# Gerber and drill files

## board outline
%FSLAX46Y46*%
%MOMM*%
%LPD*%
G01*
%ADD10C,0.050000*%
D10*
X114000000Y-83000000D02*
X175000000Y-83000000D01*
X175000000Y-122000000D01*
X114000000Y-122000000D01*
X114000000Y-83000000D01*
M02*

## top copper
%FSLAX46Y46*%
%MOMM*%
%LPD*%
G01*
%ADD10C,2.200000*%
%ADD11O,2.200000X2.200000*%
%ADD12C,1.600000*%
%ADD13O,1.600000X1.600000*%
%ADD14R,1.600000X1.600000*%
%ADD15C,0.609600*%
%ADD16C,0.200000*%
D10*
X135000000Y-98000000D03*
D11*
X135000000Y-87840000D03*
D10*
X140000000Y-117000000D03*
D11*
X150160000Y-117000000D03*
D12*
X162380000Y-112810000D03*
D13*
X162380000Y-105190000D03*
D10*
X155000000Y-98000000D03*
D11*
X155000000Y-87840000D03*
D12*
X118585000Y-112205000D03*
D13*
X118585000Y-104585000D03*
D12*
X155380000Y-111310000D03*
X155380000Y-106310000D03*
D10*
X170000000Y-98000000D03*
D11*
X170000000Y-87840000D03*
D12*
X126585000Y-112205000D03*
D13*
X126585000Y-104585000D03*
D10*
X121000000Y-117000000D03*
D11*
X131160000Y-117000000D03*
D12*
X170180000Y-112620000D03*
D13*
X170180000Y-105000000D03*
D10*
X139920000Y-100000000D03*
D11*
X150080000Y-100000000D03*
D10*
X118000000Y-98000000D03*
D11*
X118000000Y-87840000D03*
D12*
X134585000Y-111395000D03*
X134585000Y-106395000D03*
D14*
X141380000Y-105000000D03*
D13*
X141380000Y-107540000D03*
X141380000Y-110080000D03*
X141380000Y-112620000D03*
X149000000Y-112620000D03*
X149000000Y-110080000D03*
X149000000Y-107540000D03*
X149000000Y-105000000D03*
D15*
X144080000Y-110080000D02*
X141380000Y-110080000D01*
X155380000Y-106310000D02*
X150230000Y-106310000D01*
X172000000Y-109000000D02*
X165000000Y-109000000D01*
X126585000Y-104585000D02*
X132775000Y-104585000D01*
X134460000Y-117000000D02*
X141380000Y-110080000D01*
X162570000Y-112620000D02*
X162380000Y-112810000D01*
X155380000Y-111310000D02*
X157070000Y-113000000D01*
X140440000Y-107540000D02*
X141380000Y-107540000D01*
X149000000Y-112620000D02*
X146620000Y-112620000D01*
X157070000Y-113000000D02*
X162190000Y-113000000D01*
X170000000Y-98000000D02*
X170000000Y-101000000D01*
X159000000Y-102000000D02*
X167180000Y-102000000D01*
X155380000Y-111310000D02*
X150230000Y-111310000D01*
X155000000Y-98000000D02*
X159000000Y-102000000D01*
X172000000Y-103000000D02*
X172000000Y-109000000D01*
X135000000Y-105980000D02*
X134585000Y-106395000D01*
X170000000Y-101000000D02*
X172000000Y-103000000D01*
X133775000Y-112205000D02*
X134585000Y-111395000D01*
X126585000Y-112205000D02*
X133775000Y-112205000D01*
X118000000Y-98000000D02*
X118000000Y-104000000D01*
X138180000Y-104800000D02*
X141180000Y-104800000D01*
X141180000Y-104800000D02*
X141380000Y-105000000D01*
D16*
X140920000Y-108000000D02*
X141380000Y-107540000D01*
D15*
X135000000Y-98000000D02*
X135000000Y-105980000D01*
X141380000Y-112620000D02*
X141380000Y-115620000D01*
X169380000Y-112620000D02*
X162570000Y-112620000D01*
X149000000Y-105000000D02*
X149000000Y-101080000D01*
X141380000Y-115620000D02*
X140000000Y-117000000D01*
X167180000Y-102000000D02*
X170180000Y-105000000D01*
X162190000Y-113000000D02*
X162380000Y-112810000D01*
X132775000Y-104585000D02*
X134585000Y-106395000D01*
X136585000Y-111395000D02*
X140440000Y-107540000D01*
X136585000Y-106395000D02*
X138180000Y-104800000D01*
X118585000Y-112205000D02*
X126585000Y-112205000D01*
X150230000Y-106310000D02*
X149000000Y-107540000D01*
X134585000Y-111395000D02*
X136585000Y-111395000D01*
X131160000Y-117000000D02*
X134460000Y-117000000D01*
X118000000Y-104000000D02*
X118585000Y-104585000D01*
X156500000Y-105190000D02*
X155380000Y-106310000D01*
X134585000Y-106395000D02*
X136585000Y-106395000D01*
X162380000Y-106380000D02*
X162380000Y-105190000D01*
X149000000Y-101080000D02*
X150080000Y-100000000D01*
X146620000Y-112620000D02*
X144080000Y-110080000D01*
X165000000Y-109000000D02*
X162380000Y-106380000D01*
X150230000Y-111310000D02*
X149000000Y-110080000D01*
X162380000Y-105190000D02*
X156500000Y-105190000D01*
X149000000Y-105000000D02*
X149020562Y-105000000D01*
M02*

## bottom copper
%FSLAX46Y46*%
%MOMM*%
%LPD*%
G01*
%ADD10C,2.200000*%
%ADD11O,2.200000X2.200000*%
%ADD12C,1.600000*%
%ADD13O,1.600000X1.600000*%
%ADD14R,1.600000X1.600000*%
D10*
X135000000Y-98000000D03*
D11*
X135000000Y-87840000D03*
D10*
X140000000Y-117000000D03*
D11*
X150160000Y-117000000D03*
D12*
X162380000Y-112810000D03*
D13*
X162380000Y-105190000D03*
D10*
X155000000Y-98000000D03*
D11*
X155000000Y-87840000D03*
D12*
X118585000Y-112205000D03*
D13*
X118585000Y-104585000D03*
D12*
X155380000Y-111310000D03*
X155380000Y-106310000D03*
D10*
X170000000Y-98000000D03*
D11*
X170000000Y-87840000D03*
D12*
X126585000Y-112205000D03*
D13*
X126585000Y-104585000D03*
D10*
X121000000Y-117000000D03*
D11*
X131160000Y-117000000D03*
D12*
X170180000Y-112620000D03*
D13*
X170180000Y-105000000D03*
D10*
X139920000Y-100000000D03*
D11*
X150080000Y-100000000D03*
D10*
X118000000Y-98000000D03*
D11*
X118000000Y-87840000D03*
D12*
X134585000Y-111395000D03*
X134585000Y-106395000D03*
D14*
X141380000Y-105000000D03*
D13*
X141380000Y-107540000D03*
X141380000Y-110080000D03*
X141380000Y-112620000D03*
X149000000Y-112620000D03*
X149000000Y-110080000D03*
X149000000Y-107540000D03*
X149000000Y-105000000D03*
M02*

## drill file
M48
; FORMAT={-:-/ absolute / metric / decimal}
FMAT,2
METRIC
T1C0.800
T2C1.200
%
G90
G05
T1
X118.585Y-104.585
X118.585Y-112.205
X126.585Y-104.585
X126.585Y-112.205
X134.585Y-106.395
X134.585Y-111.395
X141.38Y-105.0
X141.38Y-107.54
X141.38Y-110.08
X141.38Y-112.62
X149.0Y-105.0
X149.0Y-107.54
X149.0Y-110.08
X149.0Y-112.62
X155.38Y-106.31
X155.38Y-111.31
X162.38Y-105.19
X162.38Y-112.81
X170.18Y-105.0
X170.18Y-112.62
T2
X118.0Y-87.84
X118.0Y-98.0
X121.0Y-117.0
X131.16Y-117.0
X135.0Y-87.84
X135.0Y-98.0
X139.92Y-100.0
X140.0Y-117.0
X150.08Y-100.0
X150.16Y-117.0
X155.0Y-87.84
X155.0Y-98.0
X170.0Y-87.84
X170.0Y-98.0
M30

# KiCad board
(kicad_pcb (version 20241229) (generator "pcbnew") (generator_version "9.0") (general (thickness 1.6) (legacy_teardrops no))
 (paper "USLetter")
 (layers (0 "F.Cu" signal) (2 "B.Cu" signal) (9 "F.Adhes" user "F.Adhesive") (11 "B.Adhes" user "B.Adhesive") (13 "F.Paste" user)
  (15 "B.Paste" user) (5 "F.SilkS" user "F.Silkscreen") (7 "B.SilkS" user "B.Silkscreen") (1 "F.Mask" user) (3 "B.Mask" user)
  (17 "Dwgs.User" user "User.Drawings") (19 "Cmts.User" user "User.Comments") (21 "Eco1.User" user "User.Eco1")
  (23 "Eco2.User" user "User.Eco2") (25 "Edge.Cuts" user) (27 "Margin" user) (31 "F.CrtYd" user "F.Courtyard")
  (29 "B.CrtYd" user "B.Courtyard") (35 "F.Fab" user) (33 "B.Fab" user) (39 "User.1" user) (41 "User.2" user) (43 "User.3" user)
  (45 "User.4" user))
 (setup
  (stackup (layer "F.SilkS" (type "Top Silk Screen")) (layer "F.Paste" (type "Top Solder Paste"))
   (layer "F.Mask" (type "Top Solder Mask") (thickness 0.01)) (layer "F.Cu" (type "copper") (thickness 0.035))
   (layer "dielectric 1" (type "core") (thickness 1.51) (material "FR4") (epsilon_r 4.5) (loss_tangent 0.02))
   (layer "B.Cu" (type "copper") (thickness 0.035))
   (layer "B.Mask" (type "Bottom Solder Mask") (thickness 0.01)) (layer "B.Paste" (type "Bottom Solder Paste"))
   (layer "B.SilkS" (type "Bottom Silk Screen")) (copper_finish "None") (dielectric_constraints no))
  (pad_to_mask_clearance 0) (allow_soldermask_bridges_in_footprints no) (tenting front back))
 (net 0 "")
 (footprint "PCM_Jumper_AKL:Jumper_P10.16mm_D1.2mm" (layer "F.Cu") (at 135 98 90)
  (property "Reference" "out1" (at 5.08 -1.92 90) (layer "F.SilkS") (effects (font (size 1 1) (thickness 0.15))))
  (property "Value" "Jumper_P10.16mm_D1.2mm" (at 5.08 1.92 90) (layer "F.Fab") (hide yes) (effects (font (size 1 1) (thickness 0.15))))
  (pad "1" thru_hole circle (at 0 0 90) (size 2.2 2.2) (drill 1.2) (layers "*.Cu" "*.Mask") (remove_unused_layers no))
  (pad "2" thru_hole oval (at 10.16 0 90) (size 2.2 2.2) (drill 1.2) (layers "*.Cu" "*.Mask") (remove_unused_layers no)))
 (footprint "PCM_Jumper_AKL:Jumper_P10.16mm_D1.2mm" (layer "F.Cu") (at 140 117)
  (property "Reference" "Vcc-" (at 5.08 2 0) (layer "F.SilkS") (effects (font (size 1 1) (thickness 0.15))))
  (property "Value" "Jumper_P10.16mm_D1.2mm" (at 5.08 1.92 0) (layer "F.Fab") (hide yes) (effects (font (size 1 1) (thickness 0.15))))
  (pad "1" thru_hole circle (at 0 0) (size 2.2 2.2) (drill 1.2) (layers "*.Cu" "*.Mask") (remove_unused_layers no))
  (pad "2" thru_hole oval (at 10.16 0) (size 2.2 2.2) (drill 1.2) (layers "*.Cu" "*.Mask") (remove_unused_layers no)))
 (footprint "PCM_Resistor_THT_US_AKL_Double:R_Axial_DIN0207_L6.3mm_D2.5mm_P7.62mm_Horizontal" (layer "F.Cu") (at 162.38 112.81 90)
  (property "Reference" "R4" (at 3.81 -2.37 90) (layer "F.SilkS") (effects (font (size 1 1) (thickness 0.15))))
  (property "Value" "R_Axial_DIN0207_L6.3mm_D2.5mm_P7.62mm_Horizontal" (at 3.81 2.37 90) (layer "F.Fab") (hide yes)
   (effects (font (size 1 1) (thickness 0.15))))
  (pad "1" thru_hole circle (at 0 0 90) (size 1.6 1.6) (drill 0.8) (layers "*.Cu" "*.Mask") (remove_unused_layers no))
  (pad "2" thru_hole oval (at 7.62 0 90) (size 1.6 1.6) (drill 0.8) (layers "*.Cu" "*.Mask") (remove_unused_layers no)))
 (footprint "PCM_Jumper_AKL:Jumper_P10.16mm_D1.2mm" (layer "F.Cu") (at 155 98 90)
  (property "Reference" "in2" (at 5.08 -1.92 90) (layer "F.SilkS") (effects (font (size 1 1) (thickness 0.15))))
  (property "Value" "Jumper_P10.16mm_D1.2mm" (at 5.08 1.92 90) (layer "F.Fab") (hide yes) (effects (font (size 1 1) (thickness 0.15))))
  (pad "1" thru_hole circle (at 0 0 90) (size 2.2 2.2) (drill 1.2) (layers "*.Cu" "*.Mask") (remove_unused_layers no))
  (pad "2" thru_hole oval (at 10.16 0 90) (size 2.2 2.2) (drill 1.2) (layers "*.Cu" "*.Mask") (remove_unused_layers no)))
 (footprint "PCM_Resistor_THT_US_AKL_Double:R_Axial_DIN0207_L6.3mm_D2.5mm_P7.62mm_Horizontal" (layer "F.Cu") (at 118.585 112.205 90)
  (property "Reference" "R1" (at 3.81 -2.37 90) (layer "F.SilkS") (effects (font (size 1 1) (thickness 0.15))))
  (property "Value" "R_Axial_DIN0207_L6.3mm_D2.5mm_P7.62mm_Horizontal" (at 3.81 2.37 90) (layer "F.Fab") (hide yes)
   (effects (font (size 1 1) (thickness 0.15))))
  (pad "1" thru_hole circle (at 0 0 90) (size 1.6 1.6) (drill 0.8) (layers "*.Cu" "*.Mask") (remove_unused_layers no))
  (pad "2" thru_hole oval (at 7.62 0 90) (size 1.6 1.6) (drill 0.8) (layers "*.Cu" "*.Mask") (remove_unused_layers no)))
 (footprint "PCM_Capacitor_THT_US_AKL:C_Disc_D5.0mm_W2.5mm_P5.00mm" (layer "F.Cu") (at 155.38 111.31 90)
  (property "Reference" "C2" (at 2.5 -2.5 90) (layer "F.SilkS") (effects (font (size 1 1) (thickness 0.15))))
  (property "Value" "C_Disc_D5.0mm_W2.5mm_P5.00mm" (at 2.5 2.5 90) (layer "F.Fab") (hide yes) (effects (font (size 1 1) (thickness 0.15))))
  (pad "1" thru_hole circle (at 0 0 90) (size 1.6 1.6) (drill 0.8) (layers "*.Cu" "*.Mask") (remove_unused_layers no))
  (pad "2" thru_hole circle (at 5 0 90) (size 1.6 1.6) (drill 0.8) (layers "*.Cu" "*.Mask") (remove_unused_layers no)))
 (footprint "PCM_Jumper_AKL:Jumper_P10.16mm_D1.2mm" (layer "F.Cu") (at 170 98 90)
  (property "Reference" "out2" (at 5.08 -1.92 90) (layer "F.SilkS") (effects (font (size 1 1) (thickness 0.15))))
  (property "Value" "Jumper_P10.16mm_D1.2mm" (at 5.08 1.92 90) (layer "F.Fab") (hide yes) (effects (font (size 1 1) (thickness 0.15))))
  (pad "1" thru_hole circle (at 0 0 90) (size 2.2 2.2) (drill 1.2) (layers "*.Cu" "*.Mask") (remove_unused_layers no))
  (pad "2" thru_hole oval (at 10.16 0 90) (size 2.2 2.2) (drill 1.2) (layers "*.Cu" "*.Mask") (remove_unused_layers no)))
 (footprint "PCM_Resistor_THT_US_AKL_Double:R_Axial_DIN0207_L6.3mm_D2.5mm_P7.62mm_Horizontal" (layer "F.Cu") (at 126.585 112.205 90)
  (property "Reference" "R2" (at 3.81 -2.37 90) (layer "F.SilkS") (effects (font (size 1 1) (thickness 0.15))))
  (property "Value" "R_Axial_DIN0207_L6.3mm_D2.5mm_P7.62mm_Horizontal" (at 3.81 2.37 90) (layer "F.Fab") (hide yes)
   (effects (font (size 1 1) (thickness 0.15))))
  (pad "1" thru_hole circle (at 0 0 90) (size 1.6 1.6) (drill 0.8) (layers "*.Cu" "*.Mask") (remove_unused_layers no))
  (pad "2" thru_hole oval (at 7.62 0 90) (size 1.6 1.6) (drill 0.8) (layers "*.Cu" "*.Mask") (remove_unused_layers no)))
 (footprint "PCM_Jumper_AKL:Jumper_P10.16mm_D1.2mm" (layer "F.Cu") (at 121 117)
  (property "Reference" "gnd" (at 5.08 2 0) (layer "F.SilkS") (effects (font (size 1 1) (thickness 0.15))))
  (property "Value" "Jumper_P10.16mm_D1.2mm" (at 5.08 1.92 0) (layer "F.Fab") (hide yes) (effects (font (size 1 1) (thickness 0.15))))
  (pad "1" thru_hole circle (at 0 0) (size 2.2 2.2) (drill 1.2) (layers "*.Cu" "*.Mask") (remove_unused_layers no))
  (pad "2" thru_hole oval (at 10.16 0) (size 2.2 2.2) (drill 1.2) (layers "*.Cu" "*.Mask") (remove_unused_layers no)))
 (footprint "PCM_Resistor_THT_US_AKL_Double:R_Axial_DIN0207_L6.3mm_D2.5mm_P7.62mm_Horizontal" (layer "F.Cu") (at 170.18 112.62 90)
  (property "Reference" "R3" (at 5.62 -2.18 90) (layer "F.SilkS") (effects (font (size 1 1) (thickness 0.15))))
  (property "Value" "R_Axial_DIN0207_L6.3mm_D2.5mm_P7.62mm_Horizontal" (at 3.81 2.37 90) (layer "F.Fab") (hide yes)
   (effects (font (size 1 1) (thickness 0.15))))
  (pad "1" thru_hole circle (at 0 0 90) (size 1.6 1.6) (drill 0.8) (layers "*.Cu" "*.Mask") (remove_unused_layers no))
  (pad "2" thru_hole oval (at 7.62 0 90) (size 1.6 1.6) (drill 0.8) (layers "*.Cu" "*.Mask") (remove_unused_layers no)))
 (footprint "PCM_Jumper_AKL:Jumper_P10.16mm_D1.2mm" (layer "F.Cu") (at 139.92 100)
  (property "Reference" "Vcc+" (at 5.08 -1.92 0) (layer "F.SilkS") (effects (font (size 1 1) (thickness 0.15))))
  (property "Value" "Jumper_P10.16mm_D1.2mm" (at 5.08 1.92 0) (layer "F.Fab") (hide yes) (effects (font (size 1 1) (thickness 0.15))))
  (pad "1" thru_hole circle (at 0 0) (size 2.2 2.2) (drill 1.2) (layers "*.Cu" "*.Mask") (remove_unused_layers no))
  (pad "2" thru_hole oval (at 10.16 0) (size 2.2 2.2) (drill 1.2) (layers "*.Cu" "*.Mask") (remove_unused_layers no)))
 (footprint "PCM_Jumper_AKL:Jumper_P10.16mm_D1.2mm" (layer "F.Cu") (at 118 98 90)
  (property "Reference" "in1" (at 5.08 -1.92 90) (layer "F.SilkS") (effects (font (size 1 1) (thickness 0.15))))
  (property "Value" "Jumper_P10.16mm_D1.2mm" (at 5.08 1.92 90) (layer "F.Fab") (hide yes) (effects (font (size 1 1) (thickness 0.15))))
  (pad "1" thru_hole circle (at 0 0 90) (size 2.2 2.2) (drill 1.2) (layers "*.Cu" "*.Mask") (remove_unused_layers no))
  (pad "2" thru_hole oval (at 10.16 0 90) (size 2.2 2.2) (drill 1.2) (layers "*.Cu" "*.Mask") (remove_unused_layers no)))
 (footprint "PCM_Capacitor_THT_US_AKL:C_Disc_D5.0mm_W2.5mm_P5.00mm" (layer "F.Cu") (at 134.585 111.395 90)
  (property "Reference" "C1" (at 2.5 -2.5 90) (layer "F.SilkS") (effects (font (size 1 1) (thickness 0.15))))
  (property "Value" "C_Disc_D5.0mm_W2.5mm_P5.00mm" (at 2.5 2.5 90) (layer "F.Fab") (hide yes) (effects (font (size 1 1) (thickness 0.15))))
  (pad "1" thru_hole circle (at 0 0 90) (size 1.6 1.6) (drill 0.8) (layers "*.Cu" "*.Mask") (remove_unused_layers no))
  (pad "2" thru_hole circle (at 5 0 90) (size 1.6 1.6) (drill 0.8) (layers "*.Cu" "*.Mask") (remove_unused_layers no)))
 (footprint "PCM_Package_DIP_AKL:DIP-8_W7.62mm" (layer "F.Cu") (at 141.38 105)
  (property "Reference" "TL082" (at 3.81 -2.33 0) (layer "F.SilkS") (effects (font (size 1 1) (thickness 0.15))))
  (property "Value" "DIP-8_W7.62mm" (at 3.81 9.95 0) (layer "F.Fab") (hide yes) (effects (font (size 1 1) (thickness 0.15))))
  (pad "1" thru_hole rect (at 0 0) (size 1.6 1.6) (drill 0.8) (layers "*.Cu" "*.Mask") (remove_unused_layers no))
  (pad "2" thru_hole oval (at 0 2.54) (size 1.6 1.6) (drill 0.8) (layers "*.Cu" "*.Mask") (remove_unused_layers no))
  (pad "3" thru_hole oval (at 0 5.08) (size 1.6 1.6) (drill 0.8) (layers "*.Cu" "*.Mask") (remove_unused_layers no))
  (pad "4" thru_hole oval (at 0 7.62) (size 1.6 1.6) (drill 0.8) (layers "*.Cu" "*.Mask") (remove_unused_layers no))
  (pad "5" thru_hole oval (at 7.62 7.62) (size 1.6 1.6) (drill 0.8) (layers "*.Cu" "*.Mask") (remove_unused_layers no))
  (pad "6" thru_hole oval (at 7.62 5.08) (size 1.6 1.6) (drill 0.8) (layers "*.Cu" "*.Mask") (remove_unused_layers no))
  (pad "7" thru_hole oval (at 7.62 2.54) (size 1.6 1.6) (drill 0.8) (layers "*.Cu" "*.Mask") (remove_unused_layers no))
  (pad "8" thru_hole oval (at 7.62 0) (size 1.6 1.6) (drill 0.8) (layers "*.Cu" "*.Mask") (remove_unused_layers no)))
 (gr_rect (start 114 83) (end 175 122) (stroke (width 0.05) (type solid)) (fill no) (layer "Edge.Cuts"))
 (segment (start 144.08 110.08) (end 141.38 110.08) (width 0.6096) (layer "F.Cu") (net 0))
 (segment (start 155.38 106.31) (end 150.23 106.31) (width 0.6096) (layer "F.Cu") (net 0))
 (segment (start 172 109) (end 165 109) (width 0.6096) (layer "F.Cu") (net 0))
 (segment (start 126.585 104.585) (end 132.775 104.585) (width 0.6096) (layer "F.Cu") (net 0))
 (segment (start 134.46 117) (end 141.38 110.08) (width 0.6096) (layer "F.Cu") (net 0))
 (segment (start 162.57 112.62) (end 162.38 112.81) (width 0.6096) (layer "F.Cu") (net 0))
 (segment (start 155.38 111.31) (end 157.07 113) (width 0.6096) (layer "F.Cu") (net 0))
 (segment (start 140.44 107.54) (end 141.38 107.54) (width 0.6096) (layer "F.Cu") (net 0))
 (segment (start 149 112.62) (end 146.62 112.62) (width 0.6096) (layer "F.Cu") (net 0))
 (segment (start 157.07 113) (end 162.19 113) (width 0.6096) (layer "F.Cu") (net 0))
 (segment (start 170 98) (end 170 101) (width 0.6096) (layer "F.Cu") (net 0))
 (segment (start 159 102) (end 167.18 102) (width 0.6096) (layer "F.Cu") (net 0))
 (segment (start 155.38 111.31) (end 150.23 111.31) (width 0.6096) (layer "F.Cu") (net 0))
 (segment (start 155 98) (end 159 102) (width 0.6096) (layer "F.Cu") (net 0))
 (segment (start 172 103) (end 172 109) (width 0.6096) (layer "F.Cu") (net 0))
 (segment (start 135 105.98) (end 134.585 106.395) (width 0.6096) (layer "F.Cu") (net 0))
 (segment (start 170 101) (end 172 103) (width 0.6096) (layer "F.Cu") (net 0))
 (segment (start 133.775 112.205) (end 134.585 111.395) (width 0.6096) (layer "F.Cu") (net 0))
 (segment (start 126.585 112.205) (end 133.775 112.205) (width 0.6096) (layer "F.Cu") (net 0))
 (segment (start 118 98) (end 118 104) (width 0.6096) (layer "F.Cu") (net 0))
 (segment (start 138.18 104.8) (end 141.18 104.8) (width 0.6096) (layer "F.Cu") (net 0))
 (segment (start 141.18 104.8) (end 141.38 105) (width 0.6096) (layer "F.Cu") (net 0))
 (segment (start 140.92 108) (end 141.38 107.54) (width 0.2) (layer "F.Cu") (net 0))
 (segment (start 135 98) (end 135 105.98) (width 0.6096) (layer "F.Cu") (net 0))
 (segment (start 141.38 112.62) (end 141.38 115.62) (width 0.6096) (layer "F.Cu") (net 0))
 (segment (start 169.38 112.62) (end 162.57 112.62) (width 0.6096) (layer "F.Cu") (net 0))
 (segment (start 149 105) (end 149 101.08) (width 0.6096) (layer "F.Cu") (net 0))
 (segment (start 141.38 115.62) (end 140 117) (width 0.6096) (layer "F.Cu") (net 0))
 (segment (start 167.18 102) (end 170.18 105) (width 0.6096) (layer "F.Cu") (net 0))
 (segment (start 162.19 113) (end 162.38 112.81) (width 0.6096) (layer "F.Cu") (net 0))
 (segment (start 132.775 104.585) (end 134.585 106.395) (width 0.6096) (layer "F.Cu") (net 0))
 (segment (start 136.585 111.395) (end 140.44 107.54) (width 0.6096) (layer "F.Cu") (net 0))
 (segment (start 136.585 106.395) (end 138.18 104.8) (width 0.6096) (layer "F.Cu") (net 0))
 (segment (start 118.585 112.205) (end 126.585 112.205) (width 0.6096) (layer "F.Cu") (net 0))
 (segment (start 150.23 106.31) (end 149 107.54) (width 0.6096) (layer "F.Cu") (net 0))
 (segment (start 134.585 111.395) (end 136.585 111.395) (width 0.6096) (layer "F.Cu") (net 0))
 (segment (start 131.16 117) (end 134.46 117) (width 0.6096) (layer "F.Cu") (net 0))
 (segment (start 118 104) (end 118.585 104.585) (width 0.6096) (layer "F.Cu") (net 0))
 (segment (start 156.5 105.19) (end 155.38 106.31) (width 0.6096) (layer "F.Cu") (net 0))
 (segment (start 134.585 106.395) (end 136.585 106.395) (width 0.6096) (layer "F.Cu") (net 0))
 (segment (start 162.38 106.38) (end 162.38 105.19) (width 0.6096) (layer "F.Cu") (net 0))
 (segment (start 149 101.08) (end 150.08 100) (width 0.6096) (layer "F.Cu") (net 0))
 (segment (start 146.62 112.62) (end 144.08 110.08) (width 0.6096) (layer "F.Cu") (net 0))
 (segment (start 165 109) (end 162.38 106.38) (width 0.6096) (layer "F.Cu") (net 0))
 (segment (start 150.23 111.31) (end 149 110.08) (width 0.6096) (layer "F.Cu") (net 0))
 (segment (start 162.38 105.19) (end 156.5 105.19) (width 0.6096) (layer "F.Cu") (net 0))
 (segment (start 149 105) (end 149.020562 105) (width 0.6096) (layer "F.Cu") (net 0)))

